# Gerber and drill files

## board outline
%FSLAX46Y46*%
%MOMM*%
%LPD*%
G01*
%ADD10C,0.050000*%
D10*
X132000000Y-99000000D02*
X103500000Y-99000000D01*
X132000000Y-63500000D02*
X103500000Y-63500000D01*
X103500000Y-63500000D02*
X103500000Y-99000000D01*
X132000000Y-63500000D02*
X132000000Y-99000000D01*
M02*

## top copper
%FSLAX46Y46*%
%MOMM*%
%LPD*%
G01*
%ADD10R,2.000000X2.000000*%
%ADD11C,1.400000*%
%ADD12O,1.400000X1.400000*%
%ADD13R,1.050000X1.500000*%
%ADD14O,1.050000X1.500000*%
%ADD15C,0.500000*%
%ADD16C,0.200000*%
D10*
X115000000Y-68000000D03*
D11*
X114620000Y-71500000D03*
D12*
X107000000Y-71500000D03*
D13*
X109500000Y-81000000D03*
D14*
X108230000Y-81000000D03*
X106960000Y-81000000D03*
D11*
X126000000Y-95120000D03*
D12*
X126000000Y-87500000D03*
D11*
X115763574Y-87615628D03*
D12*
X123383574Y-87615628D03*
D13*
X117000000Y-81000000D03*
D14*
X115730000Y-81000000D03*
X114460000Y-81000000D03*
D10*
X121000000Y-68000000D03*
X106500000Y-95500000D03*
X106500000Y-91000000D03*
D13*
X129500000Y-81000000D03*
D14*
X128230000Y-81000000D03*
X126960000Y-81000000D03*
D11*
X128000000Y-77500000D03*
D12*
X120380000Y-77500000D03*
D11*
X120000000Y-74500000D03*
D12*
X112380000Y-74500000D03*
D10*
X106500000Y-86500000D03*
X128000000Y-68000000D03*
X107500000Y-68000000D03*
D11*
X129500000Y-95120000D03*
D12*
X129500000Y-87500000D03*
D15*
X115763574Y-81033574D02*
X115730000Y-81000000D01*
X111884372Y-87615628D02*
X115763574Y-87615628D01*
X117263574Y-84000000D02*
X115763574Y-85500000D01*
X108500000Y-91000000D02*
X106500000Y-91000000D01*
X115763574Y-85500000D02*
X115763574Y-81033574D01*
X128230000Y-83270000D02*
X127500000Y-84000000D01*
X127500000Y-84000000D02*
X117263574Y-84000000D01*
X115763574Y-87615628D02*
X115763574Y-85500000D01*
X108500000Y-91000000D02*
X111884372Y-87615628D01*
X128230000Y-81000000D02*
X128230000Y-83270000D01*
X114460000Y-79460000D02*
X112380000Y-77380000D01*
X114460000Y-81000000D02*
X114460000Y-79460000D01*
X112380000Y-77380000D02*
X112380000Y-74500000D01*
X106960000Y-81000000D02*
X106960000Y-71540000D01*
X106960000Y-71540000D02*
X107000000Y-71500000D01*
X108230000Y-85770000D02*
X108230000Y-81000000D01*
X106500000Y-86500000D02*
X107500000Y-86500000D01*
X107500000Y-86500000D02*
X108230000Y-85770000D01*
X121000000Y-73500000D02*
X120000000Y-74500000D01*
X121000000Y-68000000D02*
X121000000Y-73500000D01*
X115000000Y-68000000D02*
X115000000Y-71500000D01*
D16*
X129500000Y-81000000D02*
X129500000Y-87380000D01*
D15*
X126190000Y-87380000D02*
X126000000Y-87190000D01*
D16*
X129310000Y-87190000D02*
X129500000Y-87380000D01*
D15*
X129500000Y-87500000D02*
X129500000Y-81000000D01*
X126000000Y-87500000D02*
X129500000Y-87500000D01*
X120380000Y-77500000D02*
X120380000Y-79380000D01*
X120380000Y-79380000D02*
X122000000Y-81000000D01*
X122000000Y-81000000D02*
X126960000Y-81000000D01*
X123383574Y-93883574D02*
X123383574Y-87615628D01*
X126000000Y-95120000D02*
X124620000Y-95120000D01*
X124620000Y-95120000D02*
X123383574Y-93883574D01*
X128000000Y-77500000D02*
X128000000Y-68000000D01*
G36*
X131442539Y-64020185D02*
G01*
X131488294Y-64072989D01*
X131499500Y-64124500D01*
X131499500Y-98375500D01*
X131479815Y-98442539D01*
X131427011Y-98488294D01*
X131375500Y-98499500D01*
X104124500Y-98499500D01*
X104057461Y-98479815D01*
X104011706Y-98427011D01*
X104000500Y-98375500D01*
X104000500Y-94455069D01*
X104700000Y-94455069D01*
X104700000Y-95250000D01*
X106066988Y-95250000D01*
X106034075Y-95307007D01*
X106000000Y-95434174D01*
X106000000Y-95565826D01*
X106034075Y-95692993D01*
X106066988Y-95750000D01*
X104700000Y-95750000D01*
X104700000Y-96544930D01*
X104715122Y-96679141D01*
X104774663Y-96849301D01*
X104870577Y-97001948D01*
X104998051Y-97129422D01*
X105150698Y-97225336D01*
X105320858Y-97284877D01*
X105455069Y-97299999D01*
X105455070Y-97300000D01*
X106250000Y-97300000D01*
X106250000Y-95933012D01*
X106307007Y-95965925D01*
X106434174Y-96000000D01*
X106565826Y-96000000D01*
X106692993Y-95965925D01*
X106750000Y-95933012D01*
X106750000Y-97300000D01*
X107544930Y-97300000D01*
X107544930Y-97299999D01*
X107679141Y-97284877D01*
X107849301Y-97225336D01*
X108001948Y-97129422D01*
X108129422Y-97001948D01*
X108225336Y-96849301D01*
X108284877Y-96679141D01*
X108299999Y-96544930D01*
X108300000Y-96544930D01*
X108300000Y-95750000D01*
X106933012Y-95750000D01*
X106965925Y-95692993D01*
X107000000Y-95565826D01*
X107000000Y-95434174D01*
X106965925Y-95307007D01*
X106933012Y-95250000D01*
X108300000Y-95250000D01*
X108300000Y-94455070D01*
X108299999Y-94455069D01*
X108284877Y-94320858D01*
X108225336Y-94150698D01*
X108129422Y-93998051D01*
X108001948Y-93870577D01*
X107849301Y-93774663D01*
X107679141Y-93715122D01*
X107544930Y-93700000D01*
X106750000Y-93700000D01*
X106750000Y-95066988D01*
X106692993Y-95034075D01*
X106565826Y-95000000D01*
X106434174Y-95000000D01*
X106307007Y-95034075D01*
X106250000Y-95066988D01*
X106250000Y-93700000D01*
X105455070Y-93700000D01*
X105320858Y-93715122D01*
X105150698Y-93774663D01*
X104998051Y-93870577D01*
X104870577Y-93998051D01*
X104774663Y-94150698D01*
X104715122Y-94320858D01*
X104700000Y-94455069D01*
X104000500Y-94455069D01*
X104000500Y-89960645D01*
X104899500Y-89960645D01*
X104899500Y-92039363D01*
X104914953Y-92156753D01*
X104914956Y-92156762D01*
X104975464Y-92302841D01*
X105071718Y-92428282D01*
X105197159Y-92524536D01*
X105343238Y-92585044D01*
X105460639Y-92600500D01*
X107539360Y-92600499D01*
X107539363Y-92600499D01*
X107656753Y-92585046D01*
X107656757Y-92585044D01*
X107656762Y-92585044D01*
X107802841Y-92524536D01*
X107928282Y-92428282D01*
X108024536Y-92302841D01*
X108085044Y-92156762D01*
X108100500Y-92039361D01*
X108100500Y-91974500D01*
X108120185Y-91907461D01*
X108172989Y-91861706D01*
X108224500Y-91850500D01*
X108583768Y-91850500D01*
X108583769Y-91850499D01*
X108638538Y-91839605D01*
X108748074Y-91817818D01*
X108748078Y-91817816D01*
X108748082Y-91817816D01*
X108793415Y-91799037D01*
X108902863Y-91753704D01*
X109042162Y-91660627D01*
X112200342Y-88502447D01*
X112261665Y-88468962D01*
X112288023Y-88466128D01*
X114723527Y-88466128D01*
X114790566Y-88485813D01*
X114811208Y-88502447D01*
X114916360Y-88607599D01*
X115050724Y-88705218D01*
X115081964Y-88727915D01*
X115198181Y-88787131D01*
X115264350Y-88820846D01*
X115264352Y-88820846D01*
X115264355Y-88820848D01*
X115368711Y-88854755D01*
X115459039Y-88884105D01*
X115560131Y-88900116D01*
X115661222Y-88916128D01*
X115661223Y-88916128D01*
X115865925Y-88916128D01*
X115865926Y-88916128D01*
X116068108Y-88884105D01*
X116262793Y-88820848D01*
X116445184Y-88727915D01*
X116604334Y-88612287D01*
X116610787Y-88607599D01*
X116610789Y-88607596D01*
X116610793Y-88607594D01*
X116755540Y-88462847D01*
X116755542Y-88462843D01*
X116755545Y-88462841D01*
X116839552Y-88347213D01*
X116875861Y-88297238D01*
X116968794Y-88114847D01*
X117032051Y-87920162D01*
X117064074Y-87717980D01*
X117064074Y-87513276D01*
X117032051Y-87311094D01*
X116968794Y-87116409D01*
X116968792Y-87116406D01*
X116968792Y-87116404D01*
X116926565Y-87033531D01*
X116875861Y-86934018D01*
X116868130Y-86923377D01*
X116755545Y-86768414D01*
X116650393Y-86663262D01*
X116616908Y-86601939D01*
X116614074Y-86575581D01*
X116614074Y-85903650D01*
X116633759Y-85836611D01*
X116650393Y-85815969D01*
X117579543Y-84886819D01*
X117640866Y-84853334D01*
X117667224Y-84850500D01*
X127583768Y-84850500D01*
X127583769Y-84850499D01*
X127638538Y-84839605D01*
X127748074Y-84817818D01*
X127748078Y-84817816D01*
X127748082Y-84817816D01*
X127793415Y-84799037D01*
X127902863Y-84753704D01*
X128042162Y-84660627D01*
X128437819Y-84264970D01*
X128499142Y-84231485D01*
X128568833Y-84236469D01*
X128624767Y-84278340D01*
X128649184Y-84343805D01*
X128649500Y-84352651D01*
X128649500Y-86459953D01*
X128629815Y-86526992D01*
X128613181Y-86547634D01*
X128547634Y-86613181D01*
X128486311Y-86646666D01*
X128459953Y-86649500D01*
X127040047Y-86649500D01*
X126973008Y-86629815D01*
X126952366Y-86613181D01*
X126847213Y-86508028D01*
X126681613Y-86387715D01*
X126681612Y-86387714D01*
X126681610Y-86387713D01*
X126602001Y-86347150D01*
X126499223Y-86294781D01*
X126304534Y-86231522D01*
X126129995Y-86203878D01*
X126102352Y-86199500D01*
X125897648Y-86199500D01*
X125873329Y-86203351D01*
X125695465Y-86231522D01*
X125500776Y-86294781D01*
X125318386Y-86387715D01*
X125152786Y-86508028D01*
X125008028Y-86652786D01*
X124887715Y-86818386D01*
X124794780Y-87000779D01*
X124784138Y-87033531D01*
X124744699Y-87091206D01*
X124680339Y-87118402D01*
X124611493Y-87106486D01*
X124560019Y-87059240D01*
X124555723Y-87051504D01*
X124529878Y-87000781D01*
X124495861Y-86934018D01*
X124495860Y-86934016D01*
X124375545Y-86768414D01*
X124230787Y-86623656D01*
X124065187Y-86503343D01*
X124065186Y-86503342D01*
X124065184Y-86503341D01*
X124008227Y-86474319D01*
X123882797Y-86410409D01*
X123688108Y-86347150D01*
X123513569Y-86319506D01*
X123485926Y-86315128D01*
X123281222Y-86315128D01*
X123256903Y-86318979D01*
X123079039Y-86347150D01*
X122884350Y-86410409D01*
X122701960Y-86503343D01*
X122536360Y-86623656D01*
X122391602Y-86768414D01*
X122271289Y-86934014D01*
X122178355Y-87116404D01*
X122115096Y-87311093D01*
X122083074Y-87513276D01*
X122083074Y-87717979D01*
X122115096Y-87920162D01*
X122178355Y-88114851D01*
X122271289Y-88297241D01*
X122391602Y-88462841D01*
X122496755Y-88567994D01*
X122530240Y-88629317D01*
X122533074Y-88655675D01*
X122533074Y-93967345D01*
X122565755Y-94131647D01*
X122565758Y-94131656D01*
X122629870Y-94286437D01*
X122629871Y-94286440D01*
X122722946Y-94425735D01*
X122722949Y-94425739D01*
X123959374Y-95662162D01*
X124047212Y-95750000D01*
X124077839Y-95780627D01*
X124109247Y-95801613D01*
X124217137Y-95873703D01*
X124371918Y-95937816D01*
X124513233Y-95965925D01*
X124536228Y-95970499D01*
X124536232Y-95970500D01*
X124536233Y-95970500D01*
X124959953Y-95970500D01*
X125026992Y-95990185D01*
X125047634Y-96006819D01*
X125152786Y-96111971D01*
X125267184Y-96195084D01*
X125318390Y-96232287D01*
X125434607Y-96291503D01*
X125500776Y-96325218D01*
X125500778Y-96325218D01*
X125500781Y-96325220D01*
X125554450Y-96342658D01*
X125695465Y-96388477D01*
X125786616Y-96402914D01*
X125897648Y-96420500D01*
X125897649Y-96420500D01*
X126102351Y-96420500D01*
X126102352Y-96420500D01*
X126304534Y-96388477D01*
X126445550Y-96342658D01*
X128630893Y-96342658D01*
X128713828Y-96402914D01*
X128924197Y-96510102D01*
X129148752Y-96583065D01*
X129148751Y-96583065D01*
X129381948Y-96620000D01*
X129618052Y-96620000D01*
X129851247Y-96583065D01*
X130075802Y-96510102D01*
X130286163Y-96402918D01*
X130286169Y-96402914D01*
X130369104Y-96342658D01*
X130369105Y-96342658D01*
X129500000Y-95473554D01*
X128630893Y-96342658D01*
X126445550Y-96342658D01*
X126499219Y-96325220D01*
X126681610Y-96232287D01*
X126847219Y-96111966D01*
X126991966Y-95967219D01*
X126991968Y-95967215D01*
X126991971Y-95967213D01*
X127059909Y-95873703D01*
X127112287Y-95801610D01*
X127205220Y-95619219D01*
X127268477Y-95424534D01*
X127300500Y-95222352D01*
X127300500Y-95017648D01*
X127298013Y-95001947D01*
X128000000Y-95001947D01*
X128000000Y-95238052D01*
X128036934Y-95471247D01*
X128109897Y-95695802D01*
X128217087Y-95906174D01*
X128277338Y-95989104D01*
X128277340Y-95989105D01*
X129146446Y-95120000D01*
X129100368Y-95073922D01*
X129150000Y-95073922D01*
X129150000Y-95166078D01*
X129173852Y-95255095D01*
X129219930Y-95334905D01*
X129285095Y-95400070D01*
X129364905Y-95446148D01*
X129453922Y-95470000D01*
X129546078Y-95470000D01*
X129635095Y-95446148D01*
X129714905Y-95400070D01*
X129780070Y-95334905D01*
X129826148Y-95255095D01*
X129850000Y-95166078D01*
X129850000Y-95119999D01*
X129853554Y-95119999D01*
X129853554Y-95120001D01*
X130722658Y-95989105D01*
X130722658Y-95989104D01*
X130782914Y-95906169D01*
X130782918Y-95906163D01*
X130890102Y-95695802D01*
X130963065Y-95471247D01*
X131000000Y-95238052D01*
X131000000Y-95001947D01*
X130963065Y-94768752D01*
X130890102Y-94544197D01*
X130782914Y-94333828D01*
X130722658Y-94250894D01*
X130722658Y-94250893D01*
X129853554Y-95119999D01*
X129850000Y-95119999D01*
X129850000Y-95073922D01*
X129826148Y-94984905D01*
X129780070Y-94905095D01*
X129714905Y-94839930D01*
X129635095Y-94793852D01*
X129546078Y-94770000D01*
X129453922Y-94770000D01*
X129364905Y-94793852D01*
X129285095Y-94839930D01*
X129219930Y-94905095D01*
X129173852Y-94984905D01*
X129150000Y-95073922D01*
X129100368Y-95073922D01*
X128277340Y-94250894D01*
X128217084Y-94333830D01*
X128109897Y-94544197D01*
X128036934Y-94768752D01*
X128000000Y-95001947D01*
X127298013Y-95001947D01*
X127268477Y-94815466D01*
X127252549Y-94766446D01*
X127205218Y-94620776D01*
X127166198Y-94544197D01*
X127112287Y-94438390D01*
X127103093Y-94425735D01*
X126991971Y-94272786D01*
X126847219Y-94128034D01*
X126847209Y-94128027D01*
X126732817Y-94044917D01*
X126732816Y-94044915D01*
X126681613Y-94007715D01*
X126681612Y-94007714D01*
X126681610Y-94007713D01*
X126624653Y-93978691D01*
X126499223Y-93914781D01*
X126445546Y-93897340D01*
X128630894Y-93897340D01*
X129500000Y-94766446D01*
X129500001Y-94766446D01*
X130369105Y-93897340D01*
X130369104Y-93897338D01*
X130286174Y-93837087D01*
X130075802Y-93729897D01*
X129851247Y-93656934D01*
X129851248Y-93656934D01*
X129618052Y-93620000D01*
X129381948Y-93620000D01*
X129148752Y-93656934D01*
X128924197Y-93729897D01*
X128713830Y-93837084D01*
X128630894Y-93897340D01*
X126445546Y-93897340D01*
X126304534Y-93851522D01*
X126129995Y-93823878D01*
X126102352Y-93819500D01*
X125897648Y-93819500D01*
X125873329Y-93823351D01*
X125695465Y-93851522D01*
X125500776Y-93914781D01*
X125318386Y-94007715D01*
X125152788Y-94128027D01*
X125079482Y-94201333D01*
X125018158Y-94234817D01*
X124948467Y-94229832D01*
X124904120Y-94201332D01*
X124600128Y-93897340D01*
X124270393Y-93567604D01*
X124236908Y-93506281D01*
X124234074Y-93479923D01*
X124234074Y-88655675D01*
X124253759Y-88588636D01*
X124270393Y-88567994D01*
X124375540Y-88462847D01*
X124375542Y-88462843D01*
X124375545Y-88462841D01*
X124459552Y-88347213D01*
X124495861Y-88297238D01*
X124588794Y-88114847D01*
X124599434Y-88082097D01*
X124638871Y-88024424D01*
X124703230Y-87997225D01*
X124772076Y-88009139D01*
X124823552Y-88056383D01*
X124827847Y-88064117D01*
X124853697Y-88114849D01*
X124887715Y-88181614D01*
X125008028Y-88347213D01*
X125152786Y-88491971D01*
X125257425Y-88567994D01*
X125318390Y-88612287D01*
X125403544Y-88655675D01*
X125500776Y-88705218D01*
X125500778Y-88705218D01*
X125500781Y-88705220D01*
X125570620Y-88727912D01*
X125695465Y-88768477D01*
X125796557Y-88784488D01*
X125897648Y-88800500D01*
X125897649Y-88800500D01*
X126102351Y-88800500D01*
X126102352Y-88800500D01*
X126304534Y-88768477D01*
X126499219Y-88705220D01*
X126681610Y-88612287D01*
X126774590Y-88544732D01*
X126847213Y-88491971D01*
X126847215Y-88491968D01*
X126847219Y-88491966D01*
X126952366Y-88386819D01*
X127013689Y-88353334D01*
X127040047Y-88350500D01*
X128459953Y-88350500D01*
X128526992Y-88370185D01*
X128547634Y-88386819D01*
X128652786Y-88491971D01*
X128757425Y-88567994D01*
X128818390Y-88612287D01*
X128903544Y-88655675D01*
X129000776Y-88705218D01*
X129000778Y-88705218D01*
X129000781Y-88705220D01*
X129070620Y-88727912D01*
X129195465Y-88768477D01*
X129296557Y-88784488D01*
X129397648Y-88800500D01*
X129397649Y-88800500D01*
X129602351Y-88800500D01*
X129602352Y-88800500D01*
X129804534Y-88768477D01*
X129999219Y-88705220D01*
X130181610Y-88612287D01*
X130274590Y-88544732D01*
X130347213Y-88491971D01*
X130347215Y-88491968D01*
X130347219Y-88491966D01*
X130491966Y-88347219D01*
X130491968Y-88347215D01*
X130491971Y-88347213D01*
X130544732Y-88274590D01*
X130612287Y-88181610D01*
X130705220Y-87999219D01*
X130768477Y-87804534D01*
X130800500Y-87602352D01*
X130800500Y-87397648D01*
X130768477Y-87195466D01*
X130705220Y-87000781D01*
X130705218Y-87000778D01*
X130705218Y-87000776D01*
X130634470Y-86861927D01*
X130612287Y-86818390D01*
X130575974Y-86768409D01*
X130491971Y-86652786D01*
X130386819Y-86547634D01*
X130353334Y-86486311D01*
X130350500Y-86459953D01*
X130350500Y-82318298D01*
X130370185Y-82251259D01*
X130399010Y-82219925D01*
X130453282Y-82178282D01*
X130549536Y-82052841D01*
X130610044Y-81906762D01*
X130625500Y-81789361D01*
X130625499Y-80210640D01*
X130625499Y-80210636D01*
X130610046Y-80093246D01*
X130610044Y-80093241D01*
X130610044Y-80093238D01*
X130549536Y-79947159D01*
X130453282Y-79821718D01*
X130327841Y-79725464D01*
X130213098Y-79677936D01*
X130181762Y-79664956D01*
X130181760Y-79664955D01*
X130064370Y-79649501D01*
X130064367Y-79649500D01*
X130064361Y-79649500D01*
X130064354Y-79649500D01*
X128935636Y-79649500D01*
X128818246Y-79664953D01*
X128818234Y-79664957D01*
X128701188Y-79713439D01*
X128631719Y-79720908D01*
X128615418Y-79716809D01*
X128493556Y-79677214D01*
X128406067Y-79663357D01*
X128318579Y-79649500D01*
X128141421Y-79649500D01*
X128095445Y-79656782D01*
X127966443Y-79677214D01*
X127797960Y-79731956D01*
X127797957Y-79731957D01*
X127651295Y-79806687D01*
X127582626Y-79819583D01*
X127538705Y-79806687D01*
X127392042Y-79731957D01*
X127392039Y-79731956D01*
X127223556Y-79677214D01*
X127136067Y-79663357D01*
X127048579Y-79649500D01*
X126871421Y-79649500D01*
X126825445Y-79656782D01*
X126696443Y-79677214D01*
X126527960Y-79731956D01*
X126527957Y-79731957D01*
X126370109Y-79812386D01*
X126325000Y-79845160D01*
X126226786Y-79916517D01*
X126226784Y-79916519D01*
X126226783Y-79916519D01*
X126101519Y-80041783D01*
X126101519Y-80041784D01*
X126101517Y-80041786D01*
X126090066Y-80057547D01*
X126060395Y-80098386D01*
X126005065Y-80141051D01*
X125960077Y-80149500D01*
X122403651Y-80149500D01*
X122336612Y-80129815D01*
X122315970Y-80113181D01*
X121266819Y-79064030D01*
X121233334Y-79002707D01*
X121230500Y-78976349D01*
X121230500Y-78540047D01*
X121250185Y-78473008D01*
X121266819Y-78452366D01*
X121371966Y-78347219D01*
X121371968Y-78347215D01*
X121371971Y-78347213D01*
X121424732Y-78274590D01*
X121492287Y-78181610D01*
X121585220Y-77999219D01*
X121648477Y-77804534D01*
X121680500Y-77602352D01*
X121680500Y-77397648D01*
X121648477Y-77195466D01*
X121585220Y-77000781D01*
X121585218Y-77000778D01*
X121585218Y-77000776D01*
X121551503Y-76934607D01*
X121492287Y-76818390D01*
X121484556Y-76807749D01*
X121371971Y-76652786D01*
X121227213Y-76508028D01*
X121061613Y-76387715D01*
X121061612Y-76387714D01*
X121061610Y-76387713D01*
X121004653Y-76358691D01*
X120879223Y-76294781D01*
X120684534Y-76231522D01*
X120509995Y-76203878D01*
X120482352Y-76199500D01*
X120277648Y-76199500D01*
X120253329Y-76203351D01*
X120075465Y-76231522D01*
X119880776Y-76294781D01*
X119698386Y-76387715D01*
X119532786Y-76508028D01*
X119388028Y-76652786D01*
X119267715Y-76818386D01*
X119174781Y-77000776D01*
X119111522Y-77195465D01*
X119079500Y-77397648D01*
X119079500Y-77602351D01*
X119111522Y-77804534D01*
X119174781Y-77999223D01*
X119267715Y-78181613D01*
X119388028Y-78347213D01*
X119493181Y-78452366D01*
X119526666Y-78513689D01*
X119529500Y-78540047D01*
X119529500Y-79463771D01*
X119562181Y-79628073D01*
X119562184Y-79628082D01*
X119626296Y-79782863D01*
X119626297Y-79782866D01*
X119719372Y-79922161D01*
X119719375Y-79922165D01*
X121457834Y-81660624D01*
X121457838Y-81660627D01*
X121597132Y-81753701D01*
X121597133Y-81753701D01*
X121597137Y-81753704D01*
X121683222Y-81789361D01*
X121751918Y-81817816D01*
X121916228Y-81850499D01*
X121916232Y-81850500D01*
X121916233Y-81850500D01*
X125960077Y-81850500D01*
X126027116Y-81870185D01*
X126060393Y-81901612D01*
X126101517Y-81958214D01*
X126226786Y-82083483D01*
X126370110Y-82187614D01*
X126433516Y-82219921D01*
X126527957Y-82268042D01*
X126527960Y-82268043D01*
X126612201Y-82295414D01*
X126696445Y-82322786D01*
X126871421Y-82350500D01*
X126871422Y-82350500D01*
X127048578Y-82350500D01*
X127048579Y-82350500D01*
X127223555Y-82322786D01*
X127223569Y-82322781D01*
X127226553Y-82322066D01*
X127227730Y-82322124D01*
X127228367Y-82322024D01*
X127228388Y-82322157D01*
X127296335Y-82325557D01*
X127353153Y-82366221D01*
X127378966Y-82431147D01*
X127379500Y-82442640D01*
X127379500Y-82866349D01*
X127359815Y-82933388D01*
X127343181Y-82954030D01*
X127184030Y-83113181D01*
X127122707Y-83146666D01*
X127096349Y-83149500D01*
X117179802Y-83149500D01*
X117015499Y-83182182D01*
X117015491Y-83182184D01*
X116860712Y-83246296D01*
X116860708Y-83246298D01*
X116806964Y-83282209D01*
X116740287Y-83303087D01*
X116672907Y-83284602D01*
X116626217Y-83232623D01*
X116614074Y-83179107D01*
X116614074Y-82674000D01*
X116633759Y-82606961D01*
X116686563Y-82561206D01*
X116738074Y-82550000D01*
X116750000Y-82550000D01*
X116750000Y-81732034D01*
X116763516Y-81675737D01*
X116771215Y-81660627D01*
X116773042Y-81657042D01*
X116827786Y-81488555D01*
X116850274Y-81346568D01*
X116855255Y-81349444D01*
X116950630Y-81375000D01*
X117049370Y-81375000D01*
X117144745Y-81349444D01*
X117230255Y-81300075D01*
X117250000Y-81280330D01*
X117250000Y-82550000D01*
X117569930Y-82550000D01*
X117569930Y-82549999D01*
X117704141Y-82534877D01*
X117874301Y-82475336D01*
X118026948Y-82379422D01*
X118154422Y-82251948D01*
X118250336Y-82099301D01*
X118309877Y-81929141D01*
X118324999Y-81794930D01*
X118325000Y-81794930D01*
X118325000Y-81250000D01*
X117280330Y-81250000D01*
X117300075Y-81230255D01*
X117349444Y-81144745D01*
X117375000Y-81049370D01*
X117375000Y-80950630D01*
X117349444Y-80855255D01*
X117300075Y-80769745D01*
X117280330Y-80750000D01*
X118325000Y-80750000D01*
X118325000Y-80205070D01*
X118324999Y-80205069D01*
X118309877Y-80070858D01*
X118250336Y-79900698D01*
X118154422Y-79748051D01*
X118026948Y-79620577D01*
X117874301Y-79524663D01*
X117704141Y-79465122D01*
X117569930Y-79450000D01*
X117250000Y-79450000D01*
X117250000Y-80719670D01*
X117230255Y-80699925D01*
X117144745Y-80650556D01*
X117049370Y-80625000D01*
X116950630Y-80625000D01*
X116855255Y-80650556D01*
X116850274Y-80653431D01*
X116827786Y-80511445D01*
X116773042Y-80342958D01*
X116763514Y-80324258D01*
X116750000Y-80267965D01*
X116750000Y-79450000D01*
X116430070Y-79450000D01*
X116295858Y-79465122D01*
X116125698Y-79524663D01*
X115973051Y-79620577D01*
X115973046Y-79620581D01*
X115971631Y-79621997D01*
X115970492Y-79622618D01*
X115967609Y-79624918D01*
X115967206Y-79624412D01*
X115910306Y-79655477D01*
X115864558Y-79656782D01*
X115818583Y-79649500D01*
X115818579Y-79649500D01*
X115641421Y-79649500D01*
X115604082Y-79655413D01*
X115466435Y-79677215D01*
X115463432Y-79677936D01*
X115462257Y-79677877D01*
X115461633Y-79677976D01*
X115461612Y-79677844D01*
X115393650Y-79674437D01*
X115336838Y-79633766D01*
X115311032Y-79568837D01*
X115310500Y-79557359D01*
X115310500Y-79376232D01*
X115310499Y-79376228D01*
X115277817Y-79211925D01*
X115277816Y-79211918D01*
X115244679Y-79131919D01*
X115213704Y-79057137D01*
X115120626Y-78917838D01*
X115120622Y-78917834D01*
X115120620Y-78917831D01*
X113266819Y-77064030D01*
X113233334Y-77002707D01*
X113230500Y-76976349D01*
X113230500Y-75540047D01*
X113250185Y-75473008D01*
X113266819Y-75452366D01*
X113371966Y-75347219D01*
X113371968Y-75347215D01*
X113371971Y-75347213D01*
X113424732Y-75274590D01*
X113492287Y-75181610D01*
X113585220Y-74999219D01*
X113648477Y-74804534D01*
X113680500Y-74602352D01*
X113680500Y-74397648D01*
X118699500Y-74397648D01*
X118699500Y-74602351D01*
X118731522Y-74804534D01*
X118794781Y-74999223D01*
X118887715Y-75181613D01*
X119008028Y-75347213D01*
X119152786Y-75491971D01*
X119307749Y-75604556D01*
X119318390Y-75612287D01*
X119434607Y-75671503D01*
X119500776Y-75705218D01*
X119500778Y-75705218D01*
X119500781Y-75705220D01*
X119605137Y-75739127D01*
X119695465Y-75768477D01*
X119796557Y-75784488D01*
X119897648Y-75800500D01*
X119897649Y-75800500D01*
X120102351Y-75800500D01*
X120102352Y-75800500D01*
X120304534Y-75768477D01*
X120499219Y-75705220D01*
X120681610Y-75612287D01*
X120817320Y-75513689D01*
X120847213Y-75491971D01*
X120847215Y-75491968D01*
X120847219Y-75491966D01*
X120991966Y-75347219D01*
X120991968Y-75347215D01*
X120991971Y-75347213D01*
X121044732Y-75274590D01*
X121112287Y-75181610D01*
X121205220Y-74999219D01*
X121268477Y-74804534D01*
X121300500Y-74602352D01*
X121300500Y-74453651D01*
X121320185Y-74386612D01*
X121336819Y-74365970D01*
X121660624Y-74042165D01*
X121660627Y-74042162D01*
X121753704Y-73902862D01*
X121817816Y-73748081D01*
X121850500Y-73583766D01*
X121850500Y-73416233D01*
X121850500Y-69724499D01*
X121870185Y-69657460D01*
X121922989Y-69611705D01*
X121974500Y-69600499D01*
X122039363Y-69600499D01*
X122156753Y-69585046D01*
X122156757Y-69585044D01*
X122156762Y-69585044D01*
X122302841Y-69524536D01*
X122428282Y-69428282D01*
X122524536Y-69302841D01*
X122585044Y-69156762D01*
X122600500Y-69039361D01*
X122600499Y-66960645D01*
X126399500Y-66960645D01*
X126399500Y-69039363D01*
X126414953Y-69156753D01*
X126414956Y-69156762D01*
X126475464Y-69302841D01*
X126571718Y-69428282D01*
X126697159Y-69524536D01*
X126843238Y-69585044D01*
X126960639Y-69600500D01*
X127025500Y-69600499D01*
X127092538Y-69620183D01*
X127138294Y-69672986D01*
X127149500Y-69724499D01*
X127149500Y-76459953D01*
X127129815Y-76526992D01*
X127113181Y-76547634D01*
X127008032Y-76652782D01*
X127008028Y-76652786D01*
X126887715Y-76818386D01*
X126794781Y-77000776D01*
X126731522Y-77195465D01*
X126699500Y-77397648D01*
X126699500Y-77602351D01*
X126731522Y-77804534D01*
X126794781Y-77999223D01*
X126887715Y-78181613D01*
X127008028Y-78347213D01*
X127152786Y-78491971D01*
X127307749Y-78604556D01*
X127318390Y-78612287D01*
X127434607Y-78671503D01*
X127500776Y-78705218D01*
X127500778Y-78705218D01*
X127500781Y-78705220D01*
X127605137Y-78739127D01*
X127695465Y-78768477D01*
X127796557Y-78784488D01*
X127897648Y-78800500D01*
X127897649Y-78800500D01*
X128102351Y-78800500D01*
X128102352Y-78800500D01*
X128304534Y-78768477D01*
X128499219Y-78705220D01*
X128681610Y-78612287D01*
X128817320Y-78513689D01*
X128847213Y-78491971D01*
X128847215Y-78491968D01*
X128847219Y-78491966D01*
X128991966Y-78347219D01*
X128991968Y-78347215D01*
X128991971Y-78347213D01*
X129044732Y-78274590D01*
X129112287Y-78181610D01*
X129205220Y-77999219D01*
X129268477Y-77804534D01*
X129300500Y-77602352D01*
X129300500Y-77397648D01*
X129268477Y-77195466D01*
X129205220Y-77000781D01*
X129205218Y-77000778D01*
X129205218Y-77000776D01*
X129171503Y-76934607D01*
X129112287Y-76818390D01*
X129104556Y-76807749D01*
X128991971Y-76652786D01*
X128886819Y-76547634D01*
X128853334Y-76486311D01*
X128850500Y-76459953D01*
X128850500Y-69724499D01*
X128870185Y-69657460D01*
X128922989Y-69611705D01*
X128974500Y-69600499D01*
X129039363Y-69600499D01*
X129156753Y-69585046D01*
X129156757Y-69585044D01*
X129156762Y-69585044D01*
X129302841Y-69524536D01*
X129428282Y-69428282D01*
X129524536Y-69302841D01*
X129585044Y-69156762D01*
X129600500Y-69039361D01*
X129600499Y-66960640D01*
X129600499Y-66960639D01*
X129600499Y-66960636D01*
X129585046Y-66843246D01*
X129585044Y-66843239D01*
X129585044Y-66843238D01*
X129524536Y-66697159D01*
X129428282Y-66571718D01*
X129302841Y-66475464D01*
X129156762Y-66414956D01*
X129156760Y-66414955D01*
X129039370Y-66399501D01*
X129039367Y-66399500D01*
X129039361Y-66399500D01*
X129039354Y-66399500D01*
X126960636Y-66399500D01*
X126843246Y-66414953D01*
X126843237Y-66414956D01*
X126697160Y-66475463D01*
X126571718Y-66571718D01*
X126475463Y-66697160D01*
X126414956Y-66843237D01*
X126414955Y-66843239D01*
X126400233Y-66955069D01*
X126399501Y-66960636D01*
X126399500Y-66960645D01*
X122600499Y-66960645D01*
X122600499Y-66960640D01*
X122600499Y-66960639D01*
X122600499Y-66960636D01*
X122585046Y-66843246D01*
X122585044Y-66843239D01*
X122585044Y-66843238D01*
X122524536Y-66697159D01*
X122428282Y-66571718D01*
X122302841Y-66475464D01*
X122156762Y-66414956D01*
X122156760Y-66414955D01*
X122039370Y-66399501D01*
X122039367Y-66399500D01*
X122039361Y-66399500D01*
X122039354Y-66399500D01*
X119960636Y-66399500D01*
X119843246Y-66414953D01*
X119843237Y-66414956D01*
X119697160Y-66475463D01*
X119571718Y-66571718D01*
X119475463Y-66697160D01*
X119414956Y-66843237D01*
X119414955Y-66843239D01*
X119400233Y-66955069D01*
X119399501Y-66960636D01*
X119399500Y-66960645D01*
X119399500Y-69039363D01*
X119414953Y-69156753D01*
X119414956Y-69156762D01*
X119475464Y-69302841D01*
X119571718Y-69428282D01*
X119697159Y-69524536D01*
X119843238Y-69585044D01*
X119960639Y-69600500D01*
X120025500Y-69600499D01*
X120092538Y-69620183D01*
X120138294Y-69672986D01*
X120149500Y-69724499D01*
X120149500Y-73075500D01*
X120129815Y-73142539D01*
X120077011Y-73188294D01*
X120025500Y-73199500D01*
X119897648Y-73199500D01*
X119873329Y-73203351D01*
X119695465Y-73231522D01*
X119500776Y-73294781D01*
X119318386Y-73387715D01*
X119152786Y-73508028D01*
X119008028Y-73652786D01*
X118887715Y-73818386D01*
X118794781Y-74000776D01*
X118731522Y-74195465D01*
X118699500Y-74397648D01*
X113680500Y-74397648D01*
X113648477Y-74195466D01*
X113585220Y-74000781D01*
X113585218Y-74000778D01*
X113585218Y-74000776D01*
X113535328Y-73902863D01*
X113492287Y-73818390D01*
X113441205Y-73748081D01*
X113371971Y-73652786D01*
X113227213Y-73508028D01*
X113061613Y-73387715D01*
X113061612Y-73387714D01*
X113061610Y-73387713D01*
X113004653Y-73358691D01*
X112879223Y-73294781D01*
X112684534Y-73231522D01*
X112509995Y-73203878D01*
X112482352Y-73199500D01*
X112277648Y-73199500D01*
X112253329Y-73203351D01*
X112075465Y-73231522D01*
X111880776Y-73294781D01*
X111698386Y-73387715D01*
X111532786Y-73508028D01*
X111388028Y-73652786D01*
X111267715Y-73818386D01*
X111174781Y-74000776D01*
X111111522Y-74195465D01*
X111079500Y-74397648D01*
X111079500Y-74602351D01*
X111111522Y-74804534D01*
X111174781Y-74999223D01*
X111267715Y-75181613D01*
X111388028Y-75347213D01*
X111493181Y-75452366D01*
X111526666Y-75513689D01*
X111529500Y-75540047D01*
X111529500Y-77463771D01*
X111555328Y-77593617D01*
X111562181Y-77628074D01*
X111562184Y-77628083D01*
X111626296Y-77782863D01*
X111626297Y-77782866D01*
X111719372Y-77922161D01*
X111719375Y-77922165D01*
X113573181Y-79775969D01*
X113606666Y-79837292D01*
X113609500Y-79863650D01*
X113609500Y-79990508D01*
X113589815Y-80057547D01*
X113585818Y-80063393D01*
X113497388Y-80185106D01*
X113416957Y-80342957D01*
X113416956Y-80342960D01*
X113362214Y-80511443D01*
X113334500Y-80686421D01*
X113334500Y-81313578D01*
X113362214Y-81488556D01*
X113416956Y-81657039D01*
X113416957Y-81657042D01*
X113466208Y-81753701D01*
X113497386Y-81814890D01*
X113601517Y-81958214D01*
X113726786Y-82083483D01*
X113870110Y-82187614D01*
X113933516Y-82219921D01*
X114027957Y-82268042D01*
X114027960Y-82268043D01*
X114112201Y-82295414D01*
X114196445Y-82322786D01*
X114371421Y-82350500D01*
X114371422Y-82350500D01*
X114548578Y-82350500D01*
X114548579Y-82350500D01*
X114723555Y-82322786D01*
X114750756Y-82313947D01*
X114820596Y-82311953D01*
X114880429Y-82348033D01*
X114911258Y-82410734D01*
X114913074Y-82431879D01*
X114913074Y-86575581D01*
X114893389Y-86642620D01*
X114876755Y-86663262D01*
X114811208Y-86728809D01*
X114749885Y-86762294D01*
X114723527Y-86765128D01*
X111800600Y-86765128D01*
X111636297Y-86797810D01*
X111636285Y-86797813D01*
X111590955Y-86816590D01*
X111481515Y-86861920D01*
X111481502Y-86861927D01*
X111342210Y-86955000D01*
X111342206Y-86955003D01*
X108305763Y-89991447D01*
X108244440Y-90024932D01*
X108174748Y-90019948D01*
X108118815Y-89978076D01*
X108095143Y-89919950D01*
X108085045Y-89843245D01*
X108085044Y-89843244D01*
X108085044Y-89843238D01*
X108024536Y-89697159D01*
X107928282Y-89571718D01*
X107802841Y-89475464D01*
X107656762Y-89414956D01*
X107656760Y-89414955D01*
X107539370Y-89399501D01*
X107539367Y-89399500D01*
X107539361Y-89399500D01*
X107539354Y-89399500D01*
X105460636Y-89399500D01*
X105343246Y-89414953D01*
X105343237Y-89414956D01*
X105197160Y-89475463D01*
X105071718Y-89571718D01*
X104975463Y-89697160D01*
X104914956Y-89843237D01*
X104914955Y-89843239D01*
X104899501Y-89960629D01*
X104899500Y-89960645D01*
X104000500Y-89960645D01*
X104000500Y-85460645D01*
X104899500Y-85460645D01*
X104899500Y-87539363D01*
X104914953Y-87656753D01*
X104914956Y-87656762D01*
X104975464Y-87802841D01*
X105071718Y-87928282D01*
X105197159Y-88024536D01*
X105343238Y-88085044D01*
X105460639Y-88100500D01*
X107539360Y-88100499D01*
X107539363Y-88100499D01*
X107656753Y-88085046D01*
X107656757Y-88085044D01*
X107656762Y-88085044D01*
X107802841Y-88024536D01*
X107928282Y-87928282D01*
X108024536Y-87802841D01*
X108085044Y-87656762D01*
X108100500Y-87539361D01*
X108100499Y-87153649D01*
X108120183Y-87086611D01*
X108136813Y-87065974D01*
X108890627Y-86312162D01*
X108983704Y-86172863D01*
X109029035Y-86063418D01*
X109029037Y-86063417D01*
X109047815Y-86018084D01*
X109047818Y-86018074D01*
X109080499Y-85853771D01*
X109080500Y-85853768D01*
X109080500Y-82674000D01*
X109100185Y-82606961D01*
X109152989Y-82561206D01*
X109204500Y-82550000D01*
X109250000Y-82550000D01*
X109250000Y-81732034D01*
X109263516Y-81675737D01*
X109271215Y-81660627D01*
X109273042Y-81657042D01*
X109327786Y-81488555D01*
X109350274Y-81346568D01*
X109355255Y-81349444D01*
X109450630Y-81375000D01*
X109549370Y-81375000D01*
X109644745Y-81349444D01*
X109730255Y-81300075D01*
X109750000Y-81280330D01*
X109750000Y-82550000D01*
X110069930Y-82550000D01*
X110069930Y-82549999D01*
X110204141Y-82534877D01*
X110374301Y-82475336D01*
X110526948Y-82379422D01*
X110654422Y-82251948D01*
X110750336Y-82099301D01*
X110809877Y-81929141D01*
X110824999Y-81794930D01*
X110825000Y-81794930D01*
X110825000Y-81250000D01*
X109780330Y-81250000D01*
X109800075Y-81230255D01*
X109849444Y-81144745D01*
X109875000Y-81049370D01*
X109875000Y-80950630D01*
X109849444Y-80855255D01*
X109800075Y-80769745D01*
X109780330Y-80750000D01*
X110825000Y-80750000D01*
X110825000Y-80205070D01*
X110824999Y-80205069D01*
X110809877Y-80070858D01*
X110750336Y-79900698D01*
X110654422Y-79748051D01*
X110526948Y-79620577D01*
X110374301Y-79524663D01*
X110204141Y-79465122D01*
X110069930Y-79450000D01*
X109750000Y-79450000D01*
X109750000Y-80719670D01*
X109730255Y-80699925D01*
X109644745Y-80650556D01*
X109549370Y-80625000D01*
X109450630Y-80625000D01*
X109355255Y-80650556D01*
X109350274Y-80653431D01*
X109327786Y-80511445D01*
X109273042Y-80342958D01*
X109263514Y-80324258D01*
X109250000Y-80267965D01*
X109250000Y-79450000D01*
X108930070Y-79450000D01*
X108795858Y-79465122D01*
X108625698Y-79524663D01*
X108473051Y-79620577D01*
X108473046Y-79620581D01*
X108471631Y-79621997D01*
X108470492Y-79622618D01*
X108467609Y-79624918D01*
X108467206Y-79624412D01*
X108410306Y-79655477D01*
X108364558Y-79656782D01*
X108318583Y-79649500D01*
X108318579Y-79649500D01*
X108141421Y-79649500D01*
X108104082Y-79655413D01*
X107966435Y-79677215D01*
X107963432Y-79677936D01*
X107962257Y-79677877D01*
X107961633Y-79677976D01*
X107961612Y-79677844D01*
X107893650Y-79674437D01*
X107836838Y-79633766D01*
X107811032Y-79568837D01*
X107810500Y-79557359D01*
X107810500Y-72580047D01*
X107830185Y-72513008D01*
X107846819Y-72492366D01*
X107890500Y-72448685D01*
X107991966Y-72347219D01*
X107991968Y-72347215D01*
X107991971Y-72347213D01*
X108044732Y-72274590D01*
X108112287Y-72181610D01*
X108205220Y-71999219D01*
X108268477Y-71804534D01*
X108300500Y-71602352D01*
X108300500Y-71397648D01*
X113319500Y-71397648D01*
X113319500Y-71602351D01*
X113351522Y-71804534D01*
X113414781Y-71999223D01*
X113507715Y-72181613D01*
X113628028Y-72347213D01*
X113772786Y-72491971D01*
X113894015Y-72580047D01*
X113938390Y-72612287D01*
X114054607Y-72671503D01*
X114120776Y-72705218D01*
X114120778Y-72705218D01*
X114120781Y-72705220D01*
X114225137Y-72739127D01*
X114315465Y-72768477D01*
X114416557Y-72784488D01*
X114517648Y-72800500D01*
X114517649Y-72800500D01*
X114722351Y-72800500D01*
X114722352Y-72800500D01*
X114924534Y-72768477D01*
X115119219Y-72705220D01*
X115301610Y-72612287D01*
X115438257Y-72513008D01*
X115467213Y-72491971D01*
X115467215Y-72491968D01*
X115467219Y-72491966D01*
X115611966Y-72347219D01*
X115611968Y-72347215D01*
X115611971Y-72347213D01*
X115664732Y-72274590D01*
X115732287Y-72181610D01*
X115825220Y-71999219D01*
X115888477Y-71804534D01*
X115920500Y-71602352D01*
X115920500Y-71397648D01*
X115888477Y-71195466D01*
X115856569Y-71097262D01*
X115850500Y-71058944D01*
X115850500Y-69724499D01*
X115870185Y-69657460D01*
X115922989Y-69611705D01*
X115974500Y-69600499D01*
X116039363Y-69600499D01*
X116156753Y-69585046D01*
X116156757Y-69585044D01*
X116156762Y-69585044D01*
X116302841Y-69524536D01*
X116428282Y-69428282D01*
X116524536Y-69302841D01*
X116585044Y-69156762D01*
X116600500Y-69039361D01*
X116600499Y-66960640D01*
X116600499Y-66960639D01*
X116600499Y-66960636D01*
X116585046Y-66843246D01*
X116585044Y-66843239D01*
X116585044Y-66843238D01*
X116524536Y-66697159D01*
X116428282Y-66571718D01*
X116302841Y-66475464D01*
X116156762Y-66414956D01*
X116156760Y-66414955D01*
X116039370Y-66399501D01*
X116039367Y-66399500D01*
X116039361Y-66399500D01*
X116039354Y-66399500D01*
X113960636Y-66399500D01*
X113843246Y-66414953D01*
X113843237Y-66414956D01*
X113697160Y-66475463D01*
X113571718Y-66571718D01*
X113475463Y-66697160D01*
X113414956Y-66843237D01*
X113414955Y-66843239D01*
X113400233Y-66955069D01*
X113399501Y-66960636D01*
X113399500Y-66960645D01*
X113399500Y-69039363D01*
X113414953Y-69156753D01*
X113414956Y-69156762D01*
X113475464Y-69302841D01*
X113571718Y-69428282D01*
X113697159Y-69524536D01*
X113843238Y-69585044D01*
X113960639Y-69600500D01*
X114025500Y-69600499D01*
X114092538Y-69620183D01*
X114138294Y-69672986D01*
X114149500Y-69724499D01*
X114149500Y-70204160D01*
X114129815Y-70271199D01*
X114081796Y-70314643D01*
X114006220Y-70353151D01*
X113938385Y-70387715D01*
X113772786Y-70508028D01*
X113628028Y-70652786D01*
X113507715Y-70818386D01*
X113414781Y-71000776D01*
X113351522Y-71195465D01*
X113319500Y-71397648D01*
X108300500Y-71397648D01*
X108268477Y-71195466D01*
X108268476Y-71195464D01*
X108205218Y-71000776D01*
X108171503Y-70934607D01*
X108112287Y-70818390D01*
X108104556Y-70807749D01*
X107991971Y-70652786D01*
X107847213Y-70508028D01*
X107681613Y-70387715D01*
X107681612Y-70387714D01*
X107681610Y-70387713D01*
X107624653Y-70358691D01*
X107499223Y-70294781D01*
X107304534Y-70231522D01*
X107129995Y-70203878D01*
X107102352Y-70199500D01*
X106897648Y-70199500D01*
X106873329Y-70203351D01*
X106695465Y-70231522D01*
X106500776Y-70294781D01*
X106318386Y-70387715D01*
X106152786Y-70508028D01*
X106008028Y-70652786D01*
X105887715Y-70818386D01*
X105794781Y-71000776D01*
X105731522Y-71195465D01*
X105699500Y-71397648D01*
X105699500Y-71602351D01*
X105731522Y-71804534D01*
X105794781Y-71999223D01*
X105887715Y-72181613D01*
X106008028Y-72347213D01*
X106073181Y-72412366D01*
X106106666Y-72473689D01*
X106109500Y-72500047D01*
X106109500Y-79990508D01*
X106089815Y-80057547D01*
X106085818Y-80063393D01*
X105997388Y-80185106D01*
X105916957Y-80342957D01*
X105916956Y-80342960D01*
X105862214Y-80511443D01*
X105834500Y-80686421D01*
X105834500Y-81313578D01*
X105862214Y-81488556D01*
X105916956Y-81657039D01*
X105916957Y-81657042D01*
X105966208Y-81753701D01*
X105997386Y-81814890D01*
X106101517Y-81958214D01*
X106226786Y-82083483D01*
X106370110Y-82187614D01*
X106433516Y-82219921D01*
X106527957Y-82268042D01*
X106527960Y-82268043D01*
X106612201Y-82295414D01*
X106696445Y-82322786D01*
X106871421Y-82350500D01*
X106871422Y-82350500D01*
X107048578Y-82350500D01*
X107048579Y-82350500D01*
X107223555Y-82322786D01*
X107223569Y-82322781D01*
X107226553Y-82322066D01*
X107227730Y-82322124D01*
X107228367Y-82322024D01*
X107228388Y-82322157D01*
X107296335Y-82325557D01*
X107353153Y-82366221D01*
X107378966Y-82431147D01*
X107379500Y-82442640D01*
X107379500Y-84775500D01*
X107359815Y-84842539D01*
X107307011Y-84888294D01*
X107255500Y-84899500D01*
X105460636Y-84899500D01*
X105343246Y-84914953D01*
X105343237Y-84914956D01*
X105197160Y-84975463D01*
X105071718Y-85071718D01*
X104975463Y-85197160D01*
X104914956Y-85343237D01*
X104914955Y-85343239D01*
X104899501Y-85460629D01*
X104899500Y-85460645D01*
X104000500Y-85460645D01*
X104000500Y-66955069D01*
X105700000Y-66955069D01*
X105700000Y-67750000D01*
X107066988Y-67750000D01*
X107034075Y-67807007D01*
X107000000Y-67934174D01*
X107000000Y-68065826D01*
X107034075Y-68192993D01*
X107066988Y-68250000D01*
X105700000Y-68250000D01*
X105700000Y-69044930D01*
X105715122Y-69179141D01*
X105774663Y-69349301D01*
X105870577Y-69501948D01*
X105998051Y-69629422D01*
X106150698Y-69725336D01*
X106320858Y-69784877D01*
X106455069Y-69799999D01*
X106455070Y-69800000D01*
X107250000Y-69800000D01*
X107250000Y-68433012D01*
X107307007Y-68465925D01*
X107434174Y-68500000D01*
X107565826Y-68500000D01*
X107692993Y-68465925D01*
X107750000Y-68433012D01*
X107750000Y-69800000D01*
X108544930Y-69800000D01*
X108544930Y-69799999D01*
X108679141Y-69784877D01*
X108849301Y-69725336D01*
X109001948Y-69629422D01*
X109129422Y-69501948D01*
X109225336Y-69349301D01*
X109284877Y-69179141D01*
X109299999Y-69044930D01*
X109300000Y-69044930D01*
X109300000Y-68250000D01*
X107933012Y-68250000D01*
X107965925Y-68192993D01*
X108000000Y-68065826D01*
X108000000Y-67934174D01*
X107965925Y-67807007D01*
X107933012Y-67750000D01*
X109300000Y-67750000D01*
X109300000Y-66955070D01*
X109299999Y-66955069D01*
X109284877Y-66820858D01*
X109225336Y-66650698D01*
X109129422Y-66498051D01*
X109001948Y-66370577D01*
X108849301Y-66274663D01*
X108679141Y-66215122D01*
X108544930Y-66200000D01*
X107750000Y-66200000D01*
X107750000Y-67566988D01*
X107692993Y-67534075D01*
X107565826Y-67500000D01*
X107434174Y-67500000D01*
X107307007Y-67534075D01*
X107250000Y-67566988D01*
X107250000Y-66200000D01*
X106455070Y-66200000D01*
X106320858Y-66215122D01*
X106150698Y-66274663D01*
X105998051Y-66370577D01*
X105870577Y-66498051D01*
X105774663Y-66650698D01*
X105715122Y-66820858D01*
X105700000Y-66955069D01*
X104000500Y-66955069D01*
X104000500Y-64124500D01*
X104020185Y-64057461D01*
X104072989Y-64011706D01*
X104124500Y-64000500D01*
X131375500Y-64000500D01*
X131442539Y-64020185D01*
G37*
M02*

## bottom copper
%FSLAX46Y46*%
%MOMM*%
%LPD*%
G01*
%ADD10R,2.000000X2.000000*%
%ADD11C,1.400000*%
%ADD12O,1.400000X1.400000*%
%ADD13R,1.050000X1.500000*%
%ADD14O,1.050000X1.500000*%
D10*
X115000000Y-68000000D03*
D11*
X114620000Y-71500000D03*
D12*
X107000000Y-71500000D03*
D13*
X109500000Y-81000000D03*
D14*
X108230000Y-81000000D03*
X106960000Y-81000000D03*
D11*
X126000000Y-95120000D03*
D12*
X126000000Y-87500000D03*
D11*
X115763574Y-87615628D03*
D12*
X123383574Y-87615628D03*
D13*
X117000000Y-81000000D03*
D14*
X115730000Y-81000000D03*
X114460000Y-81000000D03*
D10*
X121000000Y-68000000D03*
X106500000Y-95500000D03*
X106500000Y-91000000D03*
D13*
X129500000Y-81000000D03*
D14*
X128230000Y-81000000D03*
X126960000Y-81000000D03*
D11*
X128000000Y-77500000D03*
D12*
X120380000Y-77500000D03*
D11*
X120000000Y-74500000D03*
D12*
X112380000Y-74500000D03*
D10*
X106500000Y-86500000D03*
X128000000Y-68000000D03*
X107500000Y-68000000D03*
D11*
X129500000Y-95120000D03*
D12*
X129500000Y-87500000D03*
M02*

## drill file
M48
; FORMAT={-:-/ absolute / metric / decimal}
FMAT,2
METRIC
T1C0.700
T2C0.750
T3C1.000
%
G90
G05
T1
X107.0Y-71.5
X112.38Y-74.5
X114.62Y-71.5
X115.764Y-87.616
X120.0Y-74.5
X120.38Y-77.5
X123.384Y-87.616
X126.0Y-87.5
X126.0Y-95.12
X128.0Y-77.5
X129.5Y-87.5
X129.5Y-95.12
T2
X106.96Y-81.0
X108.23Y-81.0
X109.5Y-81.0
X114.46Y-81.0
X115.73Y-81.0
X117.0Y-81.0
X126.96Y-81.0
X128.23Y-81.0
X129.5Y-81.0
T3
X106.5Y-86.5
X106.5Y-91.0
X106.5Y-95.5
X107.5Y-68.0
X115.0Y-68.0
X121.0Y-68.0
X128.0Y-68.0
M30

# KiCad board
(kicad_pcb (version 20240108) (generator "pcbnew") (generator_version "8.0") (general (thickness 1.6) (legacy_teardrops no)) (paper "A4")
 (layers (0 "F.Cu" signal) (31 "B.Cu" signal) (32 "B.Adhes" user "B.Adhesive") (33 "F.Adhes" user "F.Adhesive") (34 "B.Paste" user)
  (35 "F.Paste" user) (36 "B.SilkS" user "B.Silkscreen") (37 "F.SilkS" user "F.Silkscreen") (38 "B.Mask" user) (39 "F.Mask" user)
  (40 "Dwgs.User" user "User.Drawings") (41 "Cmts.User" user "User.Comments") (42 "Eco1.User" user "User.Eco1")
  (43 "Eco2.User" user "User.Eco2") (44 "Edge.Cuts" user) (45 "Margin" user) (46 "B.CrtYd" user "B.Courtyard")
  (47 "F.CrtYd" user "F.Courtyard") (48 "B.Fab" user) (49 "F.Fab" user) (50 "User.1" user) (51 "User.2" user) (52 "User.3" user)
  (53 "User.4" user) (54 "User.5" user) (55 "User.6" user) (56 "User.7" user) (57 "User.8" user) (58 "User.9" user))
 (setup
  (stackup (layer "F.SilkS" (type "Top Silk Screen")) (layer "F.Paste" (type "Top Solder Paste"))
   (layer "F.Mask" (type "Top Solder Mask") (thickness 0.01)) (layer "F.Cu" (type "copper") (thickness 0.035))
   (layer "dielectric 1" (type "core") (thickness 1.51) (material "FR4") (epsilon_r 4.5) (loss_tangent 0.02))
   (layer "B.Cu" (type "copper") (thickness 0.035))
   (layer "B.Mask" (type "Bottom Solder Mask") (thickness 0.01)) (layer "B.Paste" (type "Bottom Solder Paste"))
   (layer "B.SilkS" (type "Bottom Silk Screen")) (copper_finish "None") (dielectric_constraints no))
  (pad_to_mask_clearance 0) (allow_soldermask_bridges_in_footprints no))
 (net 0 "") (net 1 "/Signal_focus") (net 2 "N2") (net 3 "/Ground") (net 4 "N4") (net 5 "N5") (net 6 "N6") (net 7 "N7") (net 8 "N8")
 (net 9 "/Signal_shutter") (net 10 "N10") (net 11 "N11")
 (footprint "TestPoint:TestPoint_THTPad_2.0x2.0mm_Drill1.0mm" (layer "F.Cu") (at 115 68)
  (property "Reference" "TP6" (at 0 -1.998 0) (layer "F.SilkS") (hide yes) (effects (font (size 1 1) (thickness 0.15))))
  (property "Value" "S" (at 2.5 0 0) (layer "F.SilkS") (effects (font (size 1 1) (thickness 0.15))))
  (pad "1" thru_hole rect (at 0 0) (size 2 2) (drill 1) (layers "*.Cu" "*.Mask") (remove_unused_layers no) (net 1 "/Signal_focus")))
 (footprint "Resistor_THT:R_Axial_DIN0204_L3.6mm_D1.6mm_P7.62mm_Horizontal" (layer "F.Cu") (at 114.62 71.5 180)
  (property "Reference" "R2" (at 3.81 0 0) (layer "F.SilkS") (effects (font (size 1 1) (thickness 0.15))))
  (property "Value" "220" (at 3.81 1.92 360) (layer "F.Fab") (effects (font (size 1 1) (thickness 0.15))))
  (pad "1" thru_hole circle (at 0 0 180) (size 1.4 1.4) (drill 0.7) (layers "*.Cu" "*.Mask") (remove_unused_layers no)
   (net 1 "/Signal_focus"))
  (pad "2" thru_hole oval (at 7.62 0 180) (size 1.4 1.4) (drill 0.7) (layers "*.Cu" "*.Mask") (remove_unused_layers no) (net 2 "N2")))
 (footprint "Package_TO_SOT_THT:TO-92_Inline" (layer "F.Cu") (at 109.5 81 180)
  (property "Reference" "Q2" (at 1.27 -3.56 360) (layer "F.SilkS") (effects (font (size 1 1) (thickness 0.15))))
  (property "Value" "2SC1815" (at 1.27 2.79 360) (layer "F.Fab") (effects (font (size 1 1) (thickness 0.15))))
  (pad "1" thru_hole rect (at 0 0 180) (size 1.05 1.5) (drill 0.75) (layers "*.Cu" "*.Mask") (remove_unused_layers no) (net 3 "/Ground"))
  (pad "2" thru_hole oval (at 1.27 0 180) (size 1.05 1.5) (drill 0.75) (layers "*.Cu" "*.Mask") (remove_unused_layers no) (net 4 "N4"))
  (pad "3" thru_hole oval (at 2.54 0 180) (size 1.05 1.5) (drill 0.75) (layers "*.Cu" "*.Mask") (remove_unused_layers no) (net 2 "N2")))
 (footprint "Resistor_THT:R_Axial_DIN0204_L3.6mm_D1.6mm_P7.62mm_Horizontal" (layer "F.Cu") (at 126 95.12 90)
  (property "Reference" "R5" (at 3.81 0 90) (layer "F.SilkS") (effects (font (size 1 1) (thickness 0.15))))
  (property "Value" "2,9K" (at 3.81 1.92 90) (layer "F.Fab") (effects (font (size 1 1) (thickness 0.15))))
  (pad "1" thru_hole circle (at 0 0 90) (size 1.4 1.4) (drill 0.7) (layers "*.Cu" "*.Mask") (remove_unused_layers no) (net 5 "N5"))
  (pad "2" thru_hole oval (at 7.62 0 90) (size 1.4 1.4) (drill 0.7) (layers "*.Cu" "*.Mask") (remove_unused_layers no) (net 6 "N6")))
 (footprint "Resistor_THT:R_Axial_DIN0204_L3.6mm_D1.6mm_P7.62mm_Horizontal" (layer "F.Cu") (at 115.763574 87.615628)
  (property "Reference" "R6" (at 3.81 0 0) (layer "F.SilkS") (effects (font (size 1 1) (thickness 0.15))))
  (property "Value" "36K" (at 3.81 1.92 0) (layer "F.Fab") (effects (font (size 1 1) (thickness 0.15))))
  (pad "1" thru_hole circle (at 0 0) (size 1.4 1.4) (drill 0.7) (layers "*.Cu" "*.Mask") (remove_unused_layers no) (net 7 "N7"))
  (pad "2" thru_hole oval (at 7.62 0) (size 1.4 1.4) (drill 0.7) (layers "*.Cu" "*.Mask") (remove_unused_layers no) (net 5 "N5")))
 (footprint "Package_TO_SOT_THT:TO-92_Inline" (layer "F.Cu") (at 117 81 180)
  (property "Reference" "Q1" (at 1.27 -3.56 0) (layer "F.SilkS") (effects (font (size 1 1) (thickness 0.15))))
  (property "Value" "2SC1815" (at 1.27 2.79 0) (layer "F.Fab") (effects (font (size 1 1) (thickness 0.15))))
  (pad "1" thru_hole rect (at 0 0 180) (size 1.05 1.5) (drill 0.75) (layers "*.Cu" "*.Mask") (remove_unused_layers no) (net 3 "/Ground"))
  (pad "2" thru_hole oval (at 1.27 0 180) (size 1.05 1.5) (drill 0.75) (layers "*.Cu" "*.Mask") (remove_unused_layers no) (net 7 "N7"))
  (pad "3" thru_hole oval (at 2.54 0 180) (size 1.05 1.5) (drill 0.75) (layers "*.Cu" "*.Mask") (remove_unused_layers no) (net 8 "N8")))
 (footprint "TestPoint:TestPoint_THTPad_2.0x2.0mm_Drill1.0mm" (layer "F.Cu") (at 121 68)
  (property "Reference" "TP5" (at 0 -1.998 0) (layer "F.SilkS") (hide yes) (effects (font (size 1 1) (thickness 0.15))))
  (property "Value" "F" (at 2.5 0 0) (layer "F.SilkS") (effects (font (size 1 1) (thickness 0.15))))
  (pad "1" thru_hole rect (at 0 0) (size 2 2) (drill 1) (layers "*.Cu" "*.Mask") (remove_unused_layers no) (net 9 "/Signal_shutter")))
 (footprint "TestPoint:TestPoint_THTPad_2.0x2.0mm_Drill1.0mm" (layer "F.Cu") (at 106.5 95.5)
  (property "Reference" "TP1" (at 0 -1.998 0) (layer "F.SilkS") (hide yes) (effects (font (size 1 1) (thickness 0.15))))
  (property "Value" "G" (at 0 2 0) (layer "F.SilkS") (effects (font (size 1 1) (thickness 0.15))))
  (pad "1" thru_hole rect (at 0 0) (size 2 2) (drill 1) (layers "*.Cu" "*.Mask") (remove_unused_layers no) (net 3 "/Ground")))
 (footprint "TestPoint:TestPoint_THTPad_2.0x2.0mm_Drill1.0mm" (layer "F.Cu") (at 106.5 91)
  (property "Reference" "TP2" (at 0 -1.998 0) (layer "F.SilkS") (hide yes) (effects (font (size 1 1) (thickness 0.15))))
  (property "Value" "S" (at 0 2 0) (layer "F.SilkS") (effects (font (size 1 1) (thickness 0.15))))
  (pad "1" thru_hole rect (at 0 0) (size 2 2) (drill 1) (layers "*.Cu" "*.Mask") (remove_unused_layers no) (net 7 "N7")))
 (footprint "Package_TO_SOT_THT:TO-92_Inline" (layer "F.Cu") (at 129.5 81 180)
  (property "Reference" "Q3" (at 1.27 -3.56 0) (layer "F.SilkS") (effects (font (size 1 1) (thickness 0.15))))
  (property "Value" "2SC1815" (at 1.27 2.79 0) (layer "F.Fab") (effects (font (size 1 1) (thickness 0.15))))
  (pad "1" thru_hole rect (at 0 0 180) (size 1.05 1.5) (drill 0.75) (layers "*.Cu" "*.Mask") (remove_unused_layers no) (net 6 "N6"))
  (pad "2" thru_hole oval (at 1.27 0 180) (size 1.05 1.5) (drill 0.75) (layers "*.Cu" "*.Mask") (remove_unused_layers no) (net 7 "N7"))
  (pad "3" thru_hole oval (at 2.54 0 180) (size 1.05 1.5) (drill 0.75) (layers "*.Cu" "*.Mask") (remove_unused_layers no) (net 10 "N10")))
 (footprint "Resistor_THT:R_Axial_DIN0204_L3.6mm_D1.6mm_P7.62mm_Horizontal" (layer "F.Cu") (at 128 77.5 180)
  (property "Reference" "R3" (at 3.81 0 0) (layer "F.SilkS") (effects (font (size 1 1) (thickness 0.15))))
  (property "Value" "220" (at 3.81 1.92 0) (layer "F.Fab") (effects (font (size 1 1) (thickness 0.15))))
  (pad "1" thru_hole circle (at 0 0 180) (size 1.4 1.4) (drill 0.7) (layers "*.Cu" "*.Mask") (remove_unused_layers no) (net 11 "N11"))
  (pad "2" thru_hole oval (at 7.62 0 180) (size 1.4 1.4) (drill 0.7) (layers "*.Cu" "*.Mask") (remove_unused_layers no) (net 10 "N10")))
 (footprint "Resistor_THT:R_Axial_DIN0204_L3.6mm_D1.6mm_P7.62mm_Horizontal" (layer "F.Cu") (at 120 74.5 180)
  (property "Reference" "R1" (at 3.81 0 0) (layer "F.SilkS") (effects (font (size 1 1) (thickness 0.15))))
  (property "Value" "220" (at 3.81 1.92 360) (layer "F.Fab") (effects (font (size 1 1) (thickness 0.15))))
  (pad "1" thru_hole circle (at 0 0 180) (size 1.4 1.4) (drill 0.7) (layers "*.Cu" "*.Mask") (remove_unused_layers no)
   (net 9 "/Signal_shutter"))
  (pad "2" thru_hole oval (at 7.62 0 180) (size 1.4 1.4) (drill 0.7) (layers "*.Cu" "*.Mask") (remove_unused_layers no) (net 8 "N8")))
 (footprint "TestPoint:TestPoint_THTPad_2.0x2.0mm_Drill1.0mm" (layer "F.Cu") (at 106.5 86.5)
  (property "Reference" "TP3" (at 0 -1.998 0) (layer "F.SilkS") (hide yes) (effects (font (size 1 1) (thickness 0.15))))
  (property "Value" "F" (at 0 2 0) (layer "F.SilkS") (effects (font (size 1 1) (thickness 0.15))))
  (pad "1" thru_hole rect (at 0 0) (size 2 2) (drill 1) (layers "*.Cu" "*.Mask") (remove_unused_layers no) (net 4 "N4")))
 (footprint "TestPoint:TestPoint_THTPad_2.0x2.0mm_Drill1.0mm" (layer "F.Cu") (at 128 68)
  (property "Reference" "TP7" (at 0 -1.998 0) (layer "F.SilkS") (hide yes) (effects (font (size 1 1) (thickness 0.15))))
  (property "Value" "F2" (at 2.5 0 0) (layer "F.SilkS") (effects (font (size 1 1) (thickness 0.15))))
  (pad "1" thru_hole rect (at 0 0) (size 2 2) (drill 1) (layers "*.Cu" "*.Mask") (remove_unused_layers no) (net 11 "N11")))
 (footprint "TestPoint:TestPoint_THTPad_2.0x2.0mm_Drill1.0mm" (layer "F.Cu") (at 107.5 68)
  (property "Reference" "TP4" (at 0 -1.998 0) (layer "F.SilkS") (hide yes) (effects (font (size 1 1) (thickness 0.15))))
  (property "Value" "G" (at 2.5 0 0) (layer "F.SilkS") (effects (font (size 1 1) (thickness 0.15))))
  (pad "1" thru_hole rect (at 0 0) (size 2 2) (drill 1) (layers "*.Cu" "*.Mask") (remove_unused_layers no) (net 3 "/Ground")))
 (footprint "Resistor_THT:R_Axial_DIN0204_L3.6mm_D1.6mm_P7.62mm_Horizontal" (layer "F.Cu") (at 129.5 95.12 90)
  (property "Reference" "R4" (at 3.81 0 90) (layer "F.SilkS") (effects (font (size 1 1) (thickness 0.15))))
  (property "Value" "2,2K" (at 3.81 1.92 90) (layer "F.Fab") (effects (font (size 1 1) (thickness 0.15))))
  (pad "1" thru_hole circle (at 0 0 90) (size 1.4 1.4) (drill 0.7) (layers "*.Cu" "*.Mask") (remove_unused_layers no) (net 3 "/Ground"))
  (pad "2" thru_hole oval (at 7.62 0 90) (size 1.4 1.4) (drill 0.7) (layers "*.Cu" "*.Mask") (remove_unused_layers no) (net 6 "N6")))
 (gr_line (start 132 99) (end 103.5 99) (stroke (width 0.05) (type default)) (layer "Edge.Cuts"))
 (gr_line (start 132 63.5) (end 103.5 63.5) (stroke (width 0.05) (type default)) (layer "Edge.Cuts"))
 (gr_line (start 103.5 63.5) (end 103.5 99) (stroke (width 0.05) (type default)) (layer "Edge.Cuts"))
 (gr_line (start 132 63.5) (end 132 99) (stroke (width 0.05) (type default)) (layer "Edge.Cuts"))
 (segment (start 115.763574 81.033574) (end 115.73 81) (width 0.5) (layer "F.Cu") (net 7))
 (segment (start 111.884372 87.615628) (end 115.763574 87.615628) (width 0.5) (layer "F.Cu") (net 7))
 (segment (start 117.263574 84) (end 115.763574 85.5) (width 0.5) (layer "F.Cu") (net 7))
 (segment (start 108.5 91) (end 106.5 91) (width 0.5) (layer "F.Cu") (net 7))
 (segment (start 115.763574 85.5) (end 115.763574 81.033574) (width 0.5) (layer "F.Cu") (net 7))
 (segment (start 128.23 83.27) (end 127.5 84) (width 0.5) (layer "F.Cu") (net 7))
 (segment (start 127.5 84) (end 117.263574 84) (width 0.5) (layer "F.Cu") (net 7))
 (segment (start 115.763574 87.615628) (end 115.763574 85.5) (width 0.5) (layer "F.Cu") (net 7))
 (segment (start 108.5 91) (end 111.884372 87.615628) (width 0.5) (layer "F.Cu") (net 7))
 (segment (start 128.23 81) (end 128.23 83.27) (width 0.5) (layer "F.Cu") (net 7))
 (segment (start 114.46 79.46) (end 112.38 77.38) (width 0.5) (layer "F.Cu") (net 8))
 (segment (start 114.46 81) (end 114.46 79.46) (width 0.5) (layer "F.Cu") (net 8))
 (segment (start 112.38 77.38) (end 112.38 74.5) (width 0.5) (layer "F.Cu") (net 8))
 (segment (start 106.96 81) (end 106.96 71.54) (width 0.5) (layer "F.Cu") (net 2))
 (segment (start 106.96 71.54) (end 107 71.5) (width 0.5) (layer "F.Cu") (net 2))
 (segment (start 108.23 85.77) (end 108.23 81) (width 0.5) (layer "F.Cu") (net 4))
 (segment (start 106.5 86.5) (end 107.5 86.5) (width 0.5) (layer "F.Cu") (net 4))
 (segment (start 107.5 86.5) (end 108.23 85.77) (width 0.5) (layer "F.Cu") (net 4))
 (segment (start 121 73.5) (end 120 74.5) (width 0.5) (layer "F.Cu") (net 9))
 (segment (start 121 68) (end 121 73.5) (width 0.5) (layer "F.Cu") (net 9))
 (segment (start 115 68) (end 115 71.5) (width 0.5) (layer "F.Cu") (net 1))
 (segment (start 129.5 81) (end 129.5 87.38) (width 0.2) (layer "F.Cu") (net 6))
 (segment (start 126.19 87.38) (end 126 87.19) (width 0.5) (layer "F.Cu") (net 6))
 (segment (start 129.31 87.19) (end 129.5 87.38) (width 0.2) (layer "F.Cu") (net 6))
 (segment (start 129.5 87.5) (end 129.5 81) (width 0.5) (layer "F.Cu") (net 6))
 (segment (start 126 87.5) (end 129.5 87.5) (width 0.5) (layer "F.Cu") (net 6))
 (segment (start 120.38 77.5) (end 120.38 79.38) (width 0.5) (layer "F.Cu") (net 10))
 (segment (start 120.38 79.38) (end 122 81) (width 0.5) (layer "F.Cu") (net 10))
 (segment (start 122 81) (end 126.96 81) (width 0.5) (layer "F.Cu") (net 10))
 (segment (start 123.383574 93.883574) (end 123.383574 87.615628) (width 0.5) (layer "F.Cu") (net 5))
 (segment (start 126 95.12) (end 124.62 95.12) (width 0.5) (layer "F.Cu") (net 5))
 (segment (start 124.62 95.12) (end 123.383574 93.883574) (width 0.5) (layer "F.Cu") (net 5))
 (segment (start 128 77.5) (end 128 68) (width 0.5) (layer "F.Cu") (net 11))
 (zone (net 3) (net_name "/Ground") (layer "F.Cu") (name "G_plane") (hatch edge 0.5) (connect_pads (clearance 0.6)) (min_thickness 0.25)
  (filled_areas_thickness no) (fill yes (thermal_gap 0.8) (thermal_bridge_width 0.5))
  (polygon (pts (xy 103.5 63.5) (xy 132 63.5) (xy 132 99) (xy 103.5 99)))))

